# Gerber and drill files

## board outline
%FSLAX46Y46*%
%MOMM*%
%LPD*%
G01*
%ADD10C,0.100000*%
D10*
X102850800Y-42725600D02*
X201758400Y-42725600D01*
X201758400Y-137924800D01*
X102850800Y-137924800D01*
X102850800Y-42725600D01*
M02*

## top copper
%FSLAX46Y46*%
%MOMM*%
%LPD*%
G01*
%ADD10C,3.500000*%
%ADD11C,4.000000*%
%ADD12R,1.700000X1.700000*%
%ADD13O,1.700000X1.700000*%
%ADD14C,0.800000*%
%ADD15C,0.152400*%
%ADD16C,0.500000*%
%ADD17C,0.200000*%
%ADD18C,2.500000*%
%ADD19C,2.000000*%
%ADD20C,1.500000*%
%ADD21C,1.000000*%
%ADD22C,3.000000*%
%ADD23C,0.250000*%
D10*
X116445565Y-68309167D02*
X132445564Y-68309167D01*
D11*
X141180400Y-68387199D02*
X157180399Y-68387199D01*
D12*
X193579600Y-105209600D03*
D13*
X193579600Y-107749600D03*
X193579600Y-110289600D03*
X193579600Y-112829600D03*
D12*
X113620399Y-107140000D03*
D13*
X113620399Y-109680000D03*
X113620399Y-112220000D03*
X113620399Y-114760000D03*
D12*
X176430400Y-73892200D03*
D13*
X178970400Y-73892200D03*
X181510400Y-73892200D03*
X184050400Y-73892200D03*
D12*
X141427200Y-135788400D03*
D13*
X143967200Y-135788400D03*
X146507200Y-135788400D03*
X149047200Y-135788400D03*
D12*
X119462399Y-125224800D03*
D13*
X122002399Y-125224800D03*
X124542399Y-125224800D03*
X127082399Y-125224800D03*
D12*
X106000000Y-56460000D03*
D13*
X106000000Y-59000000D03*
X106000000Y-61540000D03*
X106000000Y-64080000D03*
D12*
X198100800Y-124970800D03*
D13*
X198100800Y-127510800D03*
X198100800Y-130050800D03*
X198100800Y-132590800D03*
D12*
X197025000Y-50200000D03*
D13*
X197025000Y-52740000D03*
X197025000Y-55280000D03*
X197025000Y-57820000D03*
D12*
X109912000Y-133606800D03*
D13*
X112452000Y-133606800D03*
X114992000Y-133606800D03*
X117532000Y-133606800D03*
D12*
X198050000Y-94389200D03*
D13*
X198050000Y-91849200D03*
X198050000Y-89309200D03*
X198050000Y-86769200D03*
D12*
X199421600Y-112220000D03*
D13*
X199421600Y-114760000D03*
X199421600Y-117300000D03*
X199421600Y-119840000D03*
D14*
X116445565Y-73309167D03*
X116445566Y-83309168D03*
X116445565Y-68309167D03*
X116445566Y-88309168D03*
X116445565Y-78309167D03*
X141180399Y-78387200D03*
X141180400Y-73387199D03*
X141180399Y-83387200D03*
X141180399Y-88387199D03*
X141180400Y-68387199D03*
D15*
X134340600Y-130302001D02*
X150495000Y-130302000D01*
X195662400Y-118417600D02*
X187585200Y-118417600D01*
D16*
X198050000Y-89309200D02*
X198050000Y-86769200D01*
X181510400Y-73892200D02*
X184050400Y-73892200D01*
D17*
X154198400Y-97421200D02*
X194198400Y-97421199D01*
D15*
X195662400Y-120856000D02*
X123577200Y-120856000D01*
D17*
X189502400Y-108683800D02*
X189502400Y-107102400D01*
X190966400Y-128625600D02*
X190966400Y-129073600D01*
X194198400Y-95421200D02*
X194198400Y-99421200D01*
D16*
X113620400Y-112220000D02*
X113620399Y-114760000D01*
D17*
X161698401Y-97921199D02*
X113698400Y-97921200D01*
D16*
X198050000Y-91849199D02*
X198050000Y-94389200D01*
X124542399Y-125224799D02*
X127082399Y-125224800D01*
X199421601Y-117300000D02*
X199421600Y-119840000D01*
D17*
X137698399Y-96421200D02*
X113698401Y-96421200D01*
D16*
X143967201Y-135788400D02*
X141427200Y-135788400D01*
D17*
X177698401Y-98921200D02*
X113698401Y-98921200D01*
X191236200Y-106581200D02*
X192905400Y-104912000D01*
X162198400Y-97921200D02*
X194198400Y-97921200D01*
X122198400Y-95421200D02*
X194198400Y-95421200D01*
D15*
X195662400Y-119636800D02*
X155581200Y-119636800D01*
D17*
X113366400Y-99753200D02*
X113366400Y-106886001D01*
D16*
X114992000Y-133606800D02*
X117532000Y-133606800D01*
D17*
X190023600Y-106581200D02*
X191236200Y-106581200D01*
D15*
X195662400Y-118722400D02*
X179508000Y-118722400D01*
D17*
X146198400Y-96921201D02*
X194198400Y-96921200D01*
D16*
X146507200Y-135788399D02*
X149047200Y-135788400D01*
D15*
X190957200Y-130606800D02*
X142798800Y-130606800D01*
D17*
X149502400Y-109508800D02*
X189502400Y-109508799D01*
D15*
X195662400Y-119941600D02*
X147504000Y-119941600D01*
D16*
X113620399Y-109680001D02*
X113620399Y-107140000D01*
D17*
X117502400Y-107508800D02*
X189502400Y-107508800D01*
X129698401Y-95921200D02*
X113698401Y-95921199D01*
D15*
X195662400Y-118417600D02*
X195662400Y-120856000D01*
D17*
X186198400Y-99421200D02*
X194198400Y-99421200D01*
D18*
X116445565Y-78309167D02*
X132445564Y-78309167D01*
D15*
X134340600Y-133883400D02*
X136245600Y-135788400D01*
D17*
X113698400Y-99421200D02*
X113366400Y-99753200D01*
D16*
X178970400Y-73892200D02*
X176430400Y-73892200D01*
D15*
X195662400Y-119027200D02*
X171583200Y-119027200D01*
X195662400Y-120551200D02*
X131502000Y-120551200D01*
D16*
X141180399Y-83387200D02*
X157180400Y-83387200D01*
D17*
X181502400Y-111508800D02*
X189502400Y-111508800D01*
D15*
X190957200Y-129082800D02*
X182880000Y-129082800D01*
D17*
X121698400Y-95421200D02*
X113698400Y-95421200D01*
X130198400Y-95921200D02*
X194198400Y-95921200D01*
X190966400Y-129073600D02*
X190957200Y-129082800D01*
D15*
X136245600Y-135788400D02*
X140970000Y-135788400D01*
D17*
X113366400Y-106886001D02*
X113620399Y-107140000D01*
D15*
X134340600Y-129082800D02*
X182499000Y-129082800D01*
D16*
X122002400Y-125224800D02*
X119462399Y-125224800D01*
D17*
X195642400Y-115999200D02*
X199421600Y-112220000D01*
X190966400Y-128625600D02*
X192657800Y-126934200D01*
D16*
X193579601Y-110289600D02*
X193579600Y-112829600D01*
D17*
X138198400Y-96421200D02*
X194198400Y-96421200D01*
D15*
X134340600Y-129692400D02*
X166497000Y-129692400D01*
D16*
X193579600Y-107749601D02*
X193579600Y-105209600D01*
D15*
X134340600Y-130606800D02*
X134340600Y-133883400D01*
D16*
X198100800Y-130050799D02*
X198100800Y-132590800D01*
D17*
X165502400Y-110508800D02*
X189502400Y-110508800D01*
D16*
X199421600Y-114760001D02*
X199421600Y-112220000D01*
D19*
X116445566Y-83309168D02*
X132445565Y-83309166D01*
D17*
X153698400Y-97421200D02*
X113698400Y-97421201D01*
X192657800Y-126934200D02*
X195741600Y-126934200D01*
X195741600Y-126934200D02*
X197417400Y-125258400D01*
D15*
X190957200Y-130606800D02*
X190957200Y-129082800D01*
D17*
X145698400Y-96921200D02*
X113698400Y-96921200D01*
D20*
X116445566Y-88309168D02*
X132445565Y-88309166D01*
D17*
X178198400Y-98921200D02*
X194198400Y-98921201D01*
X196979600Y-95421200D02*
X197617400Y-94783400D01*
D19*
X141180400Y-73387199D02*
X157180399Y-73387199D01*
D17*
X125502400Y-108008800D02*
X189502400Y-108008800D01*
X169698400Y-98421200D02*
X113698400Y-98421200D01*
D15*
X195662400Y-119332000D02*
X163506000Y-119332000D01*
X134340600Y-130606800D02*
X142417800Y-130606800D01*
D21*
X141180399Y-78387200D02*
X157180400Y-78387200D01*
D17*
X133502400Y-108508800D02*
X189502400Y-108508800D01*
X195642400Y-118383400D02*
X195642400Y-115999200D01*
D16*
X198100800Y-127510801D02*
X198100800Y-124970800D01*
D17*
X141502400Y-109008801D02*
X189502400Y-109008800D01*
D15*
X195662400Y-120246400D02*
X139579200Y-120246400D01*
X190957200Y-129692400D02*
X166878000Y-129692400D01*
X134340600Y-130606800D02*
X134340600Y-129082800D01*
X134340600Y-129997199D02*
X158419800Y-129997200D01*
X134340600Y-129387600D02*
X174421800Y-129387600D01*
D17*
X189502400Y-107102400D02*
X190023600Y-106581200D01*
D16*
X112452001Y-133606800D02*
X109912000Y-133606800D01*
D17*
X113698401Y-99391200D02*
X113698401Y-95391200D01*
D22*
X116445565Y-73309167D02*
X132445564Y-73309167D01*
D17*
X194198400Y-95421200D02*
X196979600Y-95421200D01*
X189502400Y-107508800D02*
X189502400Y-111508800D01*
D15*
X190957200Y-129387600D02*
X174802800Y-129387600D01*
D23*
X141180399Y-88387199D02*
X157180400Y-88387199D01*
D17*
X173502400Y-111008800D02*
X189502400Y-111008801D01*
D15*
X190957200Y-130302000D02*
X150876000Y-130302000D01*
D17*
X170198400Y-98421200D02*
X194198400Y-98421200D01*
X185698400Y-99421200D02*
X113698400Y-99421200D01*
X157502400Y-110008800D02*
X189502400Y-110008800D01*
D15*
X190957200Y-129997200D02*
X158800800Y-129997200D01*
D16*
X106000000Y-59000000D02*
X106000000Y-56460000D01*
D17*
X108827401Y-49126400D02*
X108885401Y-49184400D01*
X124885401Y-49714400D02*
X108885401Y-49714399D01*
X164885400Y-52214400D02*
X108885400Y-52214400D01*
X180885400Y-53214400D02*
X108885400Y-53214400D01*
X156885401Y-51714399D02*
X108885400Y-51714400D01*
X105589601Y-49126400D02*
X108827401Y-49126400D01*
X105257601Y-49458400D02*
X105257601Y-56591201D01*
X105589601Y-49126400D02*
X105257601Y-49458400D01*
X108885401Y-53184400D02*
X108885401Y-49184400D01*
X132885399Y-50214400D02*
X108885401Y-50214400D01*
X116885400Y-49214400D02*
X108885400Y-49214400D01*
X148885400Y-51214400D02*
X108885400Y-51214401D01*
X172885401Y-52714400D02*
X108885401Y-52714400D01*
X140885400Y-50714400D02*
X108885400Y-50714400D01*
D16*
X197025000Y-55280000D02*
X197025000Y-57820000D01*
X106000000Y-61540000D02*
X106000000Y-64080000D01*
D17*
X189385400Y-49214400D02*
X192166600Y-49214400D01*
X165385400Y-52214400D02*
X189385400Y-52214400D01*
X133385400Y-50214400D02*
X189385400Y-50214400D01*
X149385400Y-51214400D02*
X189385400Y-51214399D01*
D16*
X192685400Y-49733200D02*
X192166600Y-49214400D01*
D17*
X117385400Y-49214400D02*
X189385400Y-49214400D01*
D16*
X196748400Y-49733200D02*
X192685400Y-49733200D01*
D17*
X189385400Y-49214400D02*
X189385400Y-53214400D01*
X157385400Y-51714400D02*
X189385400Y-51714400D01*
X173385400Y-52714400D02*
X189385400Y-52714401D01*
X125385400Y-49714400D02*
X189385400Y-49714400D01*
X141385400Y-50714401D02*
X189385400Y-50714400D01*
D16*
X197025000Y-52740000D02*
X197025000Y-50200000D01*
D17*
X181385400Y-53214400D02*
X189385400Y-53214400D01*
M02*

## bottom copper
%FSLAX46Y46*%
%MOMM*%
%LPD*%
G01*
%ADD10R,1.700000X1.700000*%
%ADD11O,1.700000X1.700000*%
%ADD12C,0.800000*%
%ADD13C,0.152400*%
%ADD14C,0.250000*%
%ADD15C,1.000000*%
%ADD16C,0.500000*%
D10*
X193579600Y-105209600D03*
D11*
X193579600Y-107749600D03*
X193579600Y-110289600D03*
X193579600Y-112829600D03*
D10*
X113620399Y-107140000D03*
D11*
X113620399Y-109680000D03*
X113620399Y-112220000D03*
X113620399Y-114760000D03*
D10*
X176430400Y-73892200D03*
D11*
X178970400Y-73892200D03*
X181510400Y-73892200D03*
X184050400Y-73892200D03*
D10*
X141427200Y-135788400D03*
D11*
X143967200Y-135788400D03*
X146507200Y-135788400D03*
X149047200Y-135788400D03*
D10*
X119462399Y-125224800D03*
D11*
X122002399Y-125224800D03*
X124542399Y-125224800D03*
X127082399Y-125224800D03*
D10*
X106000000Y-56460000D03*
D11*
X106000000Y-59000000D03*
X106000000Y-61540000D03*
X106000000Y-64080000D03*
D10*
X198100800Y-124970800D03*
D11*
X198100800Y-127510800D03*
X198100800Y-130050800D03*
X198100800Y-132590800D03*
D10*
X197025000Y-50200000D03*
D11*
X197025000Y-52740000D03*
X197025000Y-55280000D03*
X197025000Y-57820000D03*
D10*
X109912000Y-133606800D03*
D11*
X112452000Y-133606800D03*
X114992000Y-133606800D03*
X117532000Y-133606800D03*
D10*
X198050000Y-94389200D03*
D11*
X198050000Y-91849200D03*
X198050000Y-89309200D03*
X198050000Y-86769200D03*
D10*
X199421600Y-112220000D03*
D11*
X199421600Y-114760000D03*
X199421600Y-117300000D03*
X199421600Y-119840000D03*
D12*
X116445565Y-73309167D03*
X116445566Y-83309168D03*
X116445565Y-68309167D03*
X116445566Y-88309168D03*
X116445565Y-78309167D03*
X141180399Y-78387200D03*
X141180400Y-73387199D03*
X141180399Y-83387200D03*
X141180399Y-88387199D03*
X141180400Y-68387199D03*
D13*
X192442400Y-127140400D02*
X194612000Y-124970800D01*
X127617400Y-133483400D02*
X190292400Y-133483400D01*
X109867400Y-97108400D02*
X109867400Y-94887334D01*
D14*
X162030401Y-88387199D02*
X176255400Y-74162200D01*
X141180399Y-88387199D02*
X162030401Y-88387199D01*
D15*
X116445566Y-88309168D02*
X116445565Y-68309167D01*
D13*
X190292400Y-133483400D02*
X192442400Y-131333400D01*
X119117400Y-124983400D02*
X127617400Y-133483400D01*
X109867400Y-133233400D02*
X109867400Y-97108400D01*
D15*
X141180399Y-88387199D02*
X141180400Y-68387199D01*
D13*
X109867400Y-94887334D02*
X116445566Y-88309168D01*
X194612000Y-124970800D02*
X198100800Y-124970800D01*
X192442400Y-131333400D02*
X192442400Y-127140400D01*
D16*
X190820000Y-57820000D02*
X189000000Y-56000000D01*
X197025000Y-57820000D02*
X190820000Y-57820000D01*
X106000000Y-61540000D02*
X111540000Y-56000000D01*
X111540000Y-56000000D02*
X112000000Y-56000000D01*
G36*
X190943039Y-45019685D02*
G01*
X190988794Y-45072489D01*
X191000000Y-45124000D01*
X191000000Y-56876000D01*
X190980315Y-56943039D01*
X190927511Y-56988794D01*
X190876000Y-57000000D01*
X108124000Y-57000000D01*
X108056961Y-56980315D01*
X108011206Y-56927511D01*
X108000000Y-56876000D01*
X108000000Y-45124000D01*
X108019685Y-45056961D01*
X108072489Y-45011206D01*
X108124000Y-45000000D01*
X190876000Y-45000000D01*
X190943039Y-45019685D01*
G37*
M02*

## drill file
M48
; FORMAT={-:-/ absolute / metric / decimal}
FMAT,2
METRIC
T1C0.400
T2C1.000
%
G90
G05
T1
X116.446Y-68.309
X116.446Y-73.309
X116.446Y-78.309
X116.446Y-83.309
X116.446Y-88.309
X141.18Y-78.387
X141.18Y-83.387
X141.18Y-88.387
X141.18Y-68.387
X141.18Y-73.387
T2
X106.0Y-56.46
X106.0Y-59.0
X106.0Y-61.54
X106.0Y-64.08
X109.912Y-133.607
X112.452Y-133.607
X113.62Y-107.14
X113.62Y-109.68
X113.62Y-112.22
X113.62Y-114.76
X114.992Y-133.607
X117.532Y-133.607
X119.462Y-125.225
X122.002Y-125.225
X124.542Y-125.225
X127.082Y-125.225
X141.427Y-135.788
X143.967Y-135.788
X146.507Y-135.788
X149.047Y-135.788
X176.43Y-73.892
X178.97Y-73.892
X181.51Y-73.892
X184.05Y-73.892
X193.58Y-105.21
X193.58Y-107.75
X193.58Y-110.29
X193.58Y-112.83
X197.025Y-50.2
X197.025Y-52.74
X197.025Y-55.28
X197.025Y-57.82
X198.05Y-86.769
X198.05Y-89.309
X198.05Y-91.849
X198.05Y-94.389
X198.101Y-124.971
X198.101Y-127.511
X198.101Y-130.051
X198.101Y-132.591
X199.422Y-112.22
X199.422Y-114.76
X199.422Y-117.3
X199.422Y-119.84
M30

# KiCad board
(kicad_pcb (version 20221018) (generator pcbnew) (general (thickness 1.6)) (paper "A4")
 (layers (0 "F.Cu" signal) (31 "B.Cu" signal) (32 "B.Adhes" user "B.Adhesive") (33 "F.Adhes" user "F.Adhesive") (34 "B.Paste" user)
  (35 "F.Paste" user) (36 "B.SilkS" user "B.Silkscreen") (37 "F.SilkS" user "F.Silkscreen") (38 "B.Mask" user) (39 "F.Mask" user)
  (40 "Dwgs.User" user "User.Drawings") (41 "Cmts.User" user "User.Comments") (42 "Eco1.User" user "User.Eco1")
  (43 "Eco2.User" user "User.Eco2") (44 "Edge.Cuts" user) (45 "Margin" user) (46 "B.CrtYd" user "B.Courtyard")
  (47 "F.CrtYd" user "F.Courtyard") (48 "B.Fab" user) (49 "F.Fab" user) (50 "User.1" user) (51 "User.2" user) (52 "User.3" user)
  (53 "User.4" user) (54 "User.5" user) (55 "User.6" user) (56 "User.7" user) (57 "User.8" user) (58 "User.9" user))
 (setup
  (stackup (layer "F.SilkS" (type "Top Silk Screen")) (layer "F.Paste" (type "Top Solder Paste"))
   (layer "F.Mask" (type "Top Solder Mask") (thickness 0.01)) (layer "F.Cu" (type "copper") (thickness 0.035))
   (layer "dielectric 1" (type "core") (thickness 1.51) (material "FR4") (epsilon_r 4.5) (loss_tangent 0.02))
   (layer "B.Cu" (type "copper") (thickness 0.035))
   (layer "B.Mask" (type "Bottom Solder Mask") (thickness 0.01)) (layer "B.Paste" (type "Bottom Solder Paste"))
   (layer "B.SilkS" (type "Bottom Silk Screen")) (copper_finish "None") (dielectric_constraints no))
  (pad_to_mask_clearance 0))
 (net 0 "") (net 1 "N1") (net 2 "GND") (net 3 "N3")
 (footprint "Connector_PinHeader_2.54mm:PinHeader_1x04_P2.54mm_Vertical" (layer "F.Cu") (at 193.5796 105.2096)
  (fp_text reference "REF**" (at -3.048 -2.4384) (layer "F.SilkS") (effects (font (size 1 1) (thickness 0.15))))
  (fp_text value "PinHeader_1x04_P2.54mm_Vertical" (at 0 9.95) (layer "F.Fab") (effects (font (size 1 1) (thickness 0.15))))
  (pad "1" thru_hole rect (at 0 0) (size 1.7 1.7) (drill 1) (layers "*.Cu" "*.Mask"))
  (pad "2" thru_hole oval (at 0 2.54) (size 1.7 1.7) (drill 1) (layers "*.Cu" "*.Mask"))
  (pad "3" thru_hole oval (at 0 5.08) (size 1.7 1.7) (drill 1) (layers "*.Cu" "*.Mask"))
  (pad "4" thru_hole oval (at 0 7.62) (size 1.7 1.7) (drill 1) (layers "*.Cu" "*.Mask")))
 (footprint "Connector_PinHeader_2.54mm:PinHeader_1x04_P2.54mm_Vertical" (layer "F.Cu") (at 113.620399 107.14)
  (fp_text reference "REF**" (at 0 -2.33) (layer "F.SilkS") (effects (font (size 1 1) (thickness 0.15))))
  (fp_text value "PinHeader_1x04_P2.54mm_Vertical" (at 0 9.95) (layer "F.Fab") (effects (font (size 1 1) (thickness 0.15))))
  (pad "1" thru_hole rect (at 0 0) (size 1.7 1.7) (drill 1) (layers "*.Cu" "*.Mask"))
  (pad "2" thru_hole oval (at 0 2.54) (size 1.7 1.7) (drill 1) (layers "*.Cu" "*.Mask"))
  (pad "3" thru_hole oval (at 0 5.08) (size 1.7 1.7) (drill 1) (layers "*.Cu" "*.Mask"))
  (pad "4" thru_hole oval (at 0 7.62) (size 1.7 1.7) (drill 1) (layers "*.Cu" "*.Mask")))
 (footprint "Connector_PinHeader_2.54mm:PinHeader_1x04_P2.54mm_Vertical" (layer "F.Cu") (at 176.4304 73.8922 90)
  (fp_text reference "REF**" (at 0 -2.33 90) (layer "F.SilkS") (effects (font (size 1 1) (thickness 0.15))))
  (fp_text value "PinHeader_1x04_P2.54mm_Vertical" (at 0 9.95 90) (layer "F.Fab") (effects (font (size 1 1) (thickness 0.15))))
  (pad "1" thru_hole rect (at 0 0 90) (size 1.7 1.7) (drill 1) (layers "*.Cu" "*.Mask"))
  (pad "2" thru_hole oval (at 0 2.54 90) (size 1.7 1.7) (drill 1) (layers "*.Cu" "*.Mask"))
  (pad "3" thru_hole oval (at 0 5.08 90) (size 1.7 1.7) (drill 1) (layers "*.Cu" "*.Mask"))
  (pad "4" thru_hole oval (at 0 7.62 90) (size 1.7 1.7) (drill 1) (layers "*.Cu" "*.Mask")))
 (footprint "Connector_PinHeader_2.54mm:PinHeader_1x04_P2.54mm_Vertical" (layer "F.Cu") (at 141.4272 135.7884 90)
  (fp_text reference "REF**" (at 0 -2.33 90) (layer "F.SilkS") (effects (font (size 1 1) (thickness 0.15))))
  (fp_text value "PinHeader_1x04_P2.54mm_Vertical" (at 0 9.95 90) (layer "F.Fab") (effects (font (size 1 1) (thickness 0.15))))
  (pad "1" thru_hole rect (at 0 0 90) (size 1.7 1.7) (drill 1) (layers "*.Cu" "*.Mask"))
  (pad "2" thru_hole oval (at 0 2.54 90) (size 1.7 1.7) (drill 1) (layers "*.Cu" "*.Mask"))
  (pad "3" thru_hole oval (at 0 5.08 90) (size 1.7 1.7) (drill 1) (layers "*.Cu" "*.Mask"))
  (pad "4" thru_hole oval (at 0 7.62 90) (size 1.7 1.7) (drill 1) (layers "*.Cu" "*.Mask")))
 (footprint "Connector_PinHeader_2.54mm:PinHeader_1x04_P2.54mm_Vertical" (layer "F.Cu") (at 119.462399 125.2248 90)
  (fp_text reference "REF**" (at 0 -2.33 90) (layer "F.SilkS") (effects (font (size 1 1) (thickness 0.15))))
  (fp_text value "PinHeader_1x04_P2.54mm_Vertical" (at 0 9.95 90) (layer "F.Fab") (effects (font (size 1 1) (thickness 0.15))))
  (pad "1" thru_hole rect (at 0 0 90) (size 1.7 1.7) (drill 1) (layers "*.Cu" "*.Mask"))
  (pad "2" thru_hole oval (at 0 2.54 90) (size 1.7 1.7) (drill 1) (layers "*.Cu" "*.Mask"))
  (pad "3" thru_hole oval (at 0 5.08 90) (size 1.7 1.7) (drill 1) (layers "*.Cu" "*.Mask"))
  (pad "4" thru_hole oval (at 0 7.62 90) (size 1.7 1.7) (drill 1) (layers "*.Cu" "*.Mask")))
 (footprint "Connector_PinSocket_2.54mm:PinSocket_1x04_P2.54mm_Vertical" (layer "F.Cu") (at 106 56.46)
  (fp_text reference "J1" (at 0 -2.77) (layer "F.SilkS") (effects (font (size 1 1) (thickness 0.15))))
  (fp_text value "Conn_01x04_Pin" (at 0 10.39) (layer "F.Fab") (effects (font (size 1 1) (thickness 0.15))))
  (pad "1" thru_hole rect (at 0 0) (size 1.7 1.7) (drill 1) (layers "*.Cu" "*.Mask") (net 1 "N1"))
  (pad "2" thru_hole oval (at 0 2.54) (size 1.7 1.7) (drill 1) (layers "*.Cu" "*.Mask") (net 1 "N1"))
  (pad "3" thru_hole oval (at 0 5.08) (size 1.7 1.7) (drill 1) (layers "*.Cu" "*.Mask") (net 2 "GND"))
  (pad "4" thru_hole oval (at 0 7.62) (size 1.7 1.7) (drill 1) (layers "*.Cu" "*.Mask") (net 2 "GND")))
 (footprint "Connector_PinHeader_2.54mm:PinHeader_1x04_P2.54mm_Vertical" (layer "F.Cu") (at 198.1008 124.9708)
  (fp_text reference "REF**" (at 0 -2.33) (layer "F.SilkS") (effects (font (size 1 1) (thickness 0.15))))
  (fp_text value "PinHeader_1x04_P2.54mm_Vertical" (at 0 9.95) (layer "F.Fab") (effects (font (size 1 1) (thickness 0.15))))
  (pad "1" thru_hole rect (at 0 0) (size 1.7 1.7) (drill 1) (layers "*.Cu" "*.Mask"))
  (pad "2" thru_hole oval (at 0 2.54) (size 1.7 1.7) (drill 1) (layers "*.Cu" "*.Mask"))
  (pad "3" thru_hole oval (at 0 5.08) (size 1.7 1.7) (drill 1) (layers "*.Cu" "*.Mask"))
  (pad "4" thru_hole oval (at 0 7.62) (size 1.7 1.7) (drill 1) (layers "*.Cu" "*.Mask")))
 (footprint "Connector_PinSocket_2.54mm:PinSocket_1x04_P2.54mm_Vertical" (layer "F.Cu") (at 197.025 50.2)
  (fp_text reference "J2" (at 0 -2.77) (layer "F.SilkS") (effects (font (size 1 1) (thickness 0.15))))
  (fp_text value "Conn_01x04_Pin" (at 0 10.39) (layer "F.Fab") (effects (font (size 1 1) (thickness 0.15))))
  (pad "1" thru_hole rect (at 0 0) (size 1.7 1.7) (drill 1) (layers "*.Cu" "*.Mask") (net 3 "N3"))
  (pad "2" thru_hole oval (at 0 2.54) (size 1.7 1.7) (drill 1) (layers "*.Cu" "*.Mask") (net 3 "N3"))
  (pad "3" thru_hole oval (at 0 5.08) (size 1.7 1.7) (drill 1) (layers "*.Cu" "*.Mask") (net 2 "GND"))
  (pad "4" thru_hole oval (at 0 7.62) (size 1.7 1.7) (drill 1) (layers "*.Cu" "*.Mask") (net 2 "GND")))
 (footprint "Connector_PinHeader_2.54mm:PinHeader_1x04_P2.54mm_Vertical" (layer "F.Cu") (at 109.912 133.6068 90)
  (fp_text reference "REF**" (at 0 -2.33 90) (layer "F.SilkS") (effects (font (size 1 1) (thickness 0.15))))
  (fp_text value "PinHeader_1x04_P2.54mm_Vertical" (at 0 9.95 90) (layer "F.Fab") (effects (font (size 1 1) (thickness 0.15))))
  (pad "1" thru_hole rect (at 0 0 90) (size 1.7 1.7) (drill 1) (layers "*.Cu" "*.Mask"))
  (pad "2" thru_hole oval (at 0 2.54 90) (size 1.7 1.7) (drill 1) (layers "*.Cu" "*.Mask"))
  (pad "3" thru_hole oval (at 0 5.08 90) (size 1.7 1.7) (drill 1) (layers "*.Cu" "*.Mask"))
  (pad "4" thru_hole oval (at 0 7.62 90) (size 1.7 1.7) (drill 1) (layers "*.Cu" "*.Mask")))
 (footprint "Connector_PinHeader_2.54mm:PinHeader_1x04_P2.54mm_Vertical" (layer "F.Cu") (at 198.05 94.3892 180)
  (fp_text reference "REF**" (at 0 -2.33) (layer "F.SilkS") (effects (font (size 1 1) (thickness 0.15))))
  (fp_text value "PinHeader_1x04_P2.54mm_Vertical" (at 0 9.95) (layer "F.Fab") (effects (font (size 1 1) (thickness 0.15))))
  (pad "1" thru_hole rect (at 0 0 180) (size 1.7 1.7) (drill 1) (layers "*.Cu" "*.Mask"))
  (pad "2" thru_hole oval (at 0 2.54 180) (size 1.7 1.7) (drill 1) (layers "*.Cu" "*.Mask"))
  (pad "3" thru_hole oval (at 0 5.08 180) (size 1.7 1.7) (drill 1) (layers "*.Cu" "*.Mask"))
  (pad "4" thru_hole oval (at 0 7.62 180) (size 1.7 1.7) (drill 1) (layers "*.Cu" "*.Mask")))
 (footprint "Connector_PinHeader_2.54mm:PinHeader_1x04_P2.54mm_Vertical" (layer "F.Cu") (at 199.4216 112.22)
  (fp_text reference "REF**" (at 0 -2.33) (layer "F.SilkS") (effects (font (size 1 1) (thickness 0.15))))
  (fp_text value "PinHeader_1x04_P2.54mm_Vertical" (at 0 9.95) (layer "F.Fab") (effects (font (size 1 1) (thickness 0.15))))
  (pad "1" thru_hole rect (at 0 0) (size 1.7 1.7) (drill 1) (layers "*.Cu" "*.Mask"))
  (pad "2" thru_hole oval (at 0 2.54) (size 1.7 1.7) (drill 1) (layers "*.Cu" "*.Mask"))
  (pad "3" thru_hole oval (at 0 5.08) (size 1.7 1.7) (drill 1) (layers "*.Cu" "*.Mask"))
  (pad "4" thru_hole oval (at 0 7.62) (size 1.7 1.7) (drill 1) (layers "*.Cu" "*.Mask")))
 (gr_line (start 116.445565 68.309167) (end 132.445564 68.309167) (stroke (width 3.5) (type default)) (layer "F.Cu"))
 (gr_line (start 141.1804 68.387199) (end 157.180399 68.387199) (stroke (width 4) (type default)) (layer "F.Cu"))
 (gr_rect (start 102.8508 42.7256) (end 201.7584 137.9248) (stroke (width 0.1) (type default)) (fill none) (layer "Edge.Cuts"))
 (segment (start 134.3406 130.302001) (end 150.495 130.302) (width 0.1524) (layer "F.Cu") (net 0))
 (segment (start 195.6624 118.4176) (end 187.5852 118.4176) (width 0.1524) (layer "F.Cu") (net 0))
 (segment (start 198.05 89.3092) (end 198.05 86.7692) (width 0.5) (layer "F.Cu") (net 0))
 (segment (start 181.5104 73.8922) (end 184.0504 73.8922) (width 0.5) (layer "F.Cu") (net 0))
 (segment (start 154.1984 97.4212) (end 194.1984 97.421199) (width 0.2) (layer "F.Cu") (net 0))
 (segment (start 195.6624 120.856) (end 123.5772 120.856) (width 0.1524) (layer "F.Cu") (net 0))
 (segment (start 189.5024 108.6838) (end 189.5024 107.1024) (width 0.2) (layer "F.Cu") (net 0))
 (segment (start 190.9664 128.6256) (end 190.9664 129.0736) (width 0.2) (layer "F.Cu") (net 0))
 (segment (start 194.1984 95.4212) (end 194.1984 99.4212) (width 0.2) (layer "F.Cu") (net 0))
 (segment (start 113.6204 112.22) (end 113.620399 114.76) (width 0.5) (layer "F.Cu") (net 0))
 (segment (start 161.698401 97.921199) (end 113.6984 97.9212) (width 0.2) (layer "F.Cu") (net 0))
 (segment (start 198.05 91.849199) (end 198.05 94.3892) (width 0.5) (layer "F.Cu") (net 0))
 (segment (start 124.542399 125.224799) (end 127.082399 125.2248) (width 0.5) (layer "F.Cu") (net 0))
 (segment (start 199.421601 117.3) (end 199.4216 119.84) (width 0.5) (layer "F.Cu") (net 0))
 (segment (start 137.698399 96.4212) (end 113.698401 96.4212) (width 0.2) (layer "F.Cu") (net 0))
 (segment (start 143.967201 135.7884) (end 141.4272 135.7884) (width 0.5) (layer "F.Cu") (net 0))
 (segment (start 177.698401 98.9212) (end 113.698401 98.9212) (width 0.2) (layer "F.Cu") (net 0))
 (segment (start 191.2362 106.5812) (end 192.9054 104.912) (width 0.2) (layer "F.Cu") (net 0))
 (segment (start 162.1984 97.9212) (end 194.1984 97.9212) (width 0.2) (layer "F.Cu") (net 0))
 (segment (start 122.1984 95.4212) (end 194.1984 95.4212) (width 0.2) (layer "F.Cu") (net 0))
 (segment (start 195.6624 119.6368) (end 155.5812 119.6368) (width 0.1524) (layer "F.Cu") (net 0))
 (segment (start 113.3664 99.7532) (end 113.3664 106.886001) (width 0.2) (layer "F.Cu") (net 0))
 (segment (start 114.992 133.6068) (end 117.532 133.6068) (width 0.5) (layer "F.Cu") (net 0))
 (segment (start 190.0236 106.5812) (end 191.2362 106.5812) (width 0.2) (layer "F.Cu") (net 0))
 (segment (start 195.6624 118.7224) (end 179.508 118.7224) (width 0.1524) (layer "F.Cu") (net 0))
 (segment (start 146.1984 96.921201) (end 194.1984 96.9212) (width 0.2) (layer "F.Cu") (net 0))
 (segment (start 146.5072 135.788399) (end 149.0472 135.7884) (width 0.5) (layer "F.Cu") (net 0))
 (segment (start 190.9572 130.6068) (end 142.7988 130.6068) (width 0.1524) (layer "F.Cu") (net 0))
 (segment (start 149.5024 109.5088) (end 189.5024 109.508799) (width 0.2) (layer "F.Cu") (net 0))
 (segment (start 195.6624 119.9416) (end 147.504 119.9416) (width 0.1524) (layer "F.Cu") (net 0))
 (segment (start 113.620399 109.680001) (end 113.620399 107.14) (width 0.5) (layer "F.Cu") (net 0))
 (segment (start 117.5024 107.5088) (end 189.5024 107.5088) (width 0.2) (layer "F.Cu") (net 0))
 (segment (start 129.698401 95.9212) (end 113.698401 95.921199) (width 0.2) (layer "F.Cu") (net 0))
 (segment (start 195.6624 118.4176) (end 195.6624 120.856) (width 0.1524) (layer "F.Cu") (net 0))
 (segment (start 186.1984 99.4212) (end 194.1984 99.4212) (width 0.2) (layer "F.Cu") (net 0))
 (segment (start 116.445565 78.309167) (end 132.445564 78.309167) (width 2.5) (layer "F.Cu") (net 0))
 (segment (start 134.3406 133.8834) (end 136.2456 135.7884) (width 0.1524) (layer "F.Cu") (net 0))
 (segment (start 113.6984 99.4212) (end 113.3664 99.7532) (width 0.2) (layer "F.Cu") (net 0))
 (segment (start 178.9704 73.8922) (end 176.4304 73.8922) (width 0.5) (layer "F.Cu") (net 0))
 (segment (start 195.6624 119.0272) (end 171.5832 119.0272) (width 0.1524) (layer "F.Cu") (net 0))
 (segment (start 195.6624 120.5512) (end 131.502 120.5512) (width 0.1524) (layer "F.Cu") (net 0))
 (segment (start 141.180399 83.3872) (end 157.1804 83.3872) (width 0.5) (layer "F.Cu") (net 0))
 (segment (start 181.5024 111.5088) (end 189.5024 111.5088) (width 0.2) (layer "F.Cu") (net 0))
 (segment (start 190.9572 129.0828) (end 182.88 129.0828) (width 0.1524) (layer "F.Cu") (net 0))
 (segment (start 121.6984 95.4212) (end 113.6984 95.4212) (width 0.2) (layer "F.Cu") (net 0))
 (segment (start 130.1984 95.9212) (end 194.1984 95.9212) (width 0.2) (layer "F.Cu") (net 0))
 (segment (start 190.9664 129.0736) (end 190.9572 129.0828) (width 0.2) (layer "F.Cu") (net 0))
 (segment (start 136.2456 135.7884) (end 140.97 135.7884) (width 0.1524) (layer "F.Cu") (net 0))
 (segment (start 113.3664 106.886001) (end 113.620399 107.14) (width 0.2) (layer "F.Cu") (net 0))
 (segment (start 134.3406 129.0828) (end 182.499 129.0828) (width 0.1524) (layer "F.Cu") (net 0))
 (segment (start 122.0024 125.2248) (end 119.462399 125.2248) (width 0.5) (layer "F.Cu") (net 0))
 (segment (start 195.6424 115.9992) (end 199.4216 112.22) (width 0.2) (layer "F.Cu") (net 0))
 (segment (start 190.9664 128.6256) (end 192.6578 126.9342) (width 0.2) (layer "F.Cu") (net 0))
 (segment (start 193.579601 110.2896) (end 193.5796 112.8296) (width 0.5) (layer "F.Cu") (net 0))
 (segment (start 138.1984 96.4212) (end 194.1984 96.4212) (width 0.2) (layer "F.Cu") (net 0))
 (segment (start 134.3406 129.6924) (end 166.497 129.6924) (width 0.1524) (layer "F.Cu") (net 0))
 (segment (start 193.5796 107.749601) (end 193.5796 105.2096) (width 0.5) (layer "F.Cu") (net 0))
 (segment (start 134.3406 130.6068) (end 134.3406 133.8834) (width 0.1524) (layer "F.Cu") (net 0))
 (segment (start 198.1008 130.050799) (end 198.1008 132.5908) (width 0.5) (layer "F.Cu") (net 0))
 (segment (start 165.5024 110.5088) (end 189.5024 110.5088) (width 0.2) (layer "F.Cu") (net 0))
 (segment (start 199.4216 114.760001) (end 199.4216 112.22) (width 0.5) (layer "F.Cu") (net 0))
 (segment (start 116.445566 83.309168) (end 132.445565 83.309166) (width 2) (layer "F.Cu") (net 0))
 (segment (start 153.6984 97.4212) (end 113.6984 97.421201) (width 0.2) (layer "F.Cu") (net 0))
 (segment (start 192.6578 126.9342) (end 195.7416 126.9342) (width 0.2) (layer "F.Cu") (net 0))
 (segment (start 195.7416 126.9342) (end 197.4174 125.2584) (width 0.2) (layer "F.Cu") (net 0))
 (segment (start 190.9572 130.6068) (end 190.9572 129.0828) (width 0.1524) (layer "F.Cu") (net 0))
 (segment (start 145.6984 96.9212) (end 113.6984 96.9212) (width 0.2) (layer "F.Cu") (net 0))
 (segment (start 116.445566 88.309168) (end 132.445565 88.309166) (width 1.5) (layer "F.Cu") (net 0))
 (segment (start 178.1984 98.9212) (end 194.1984 98.921201) (width 0.2) (layer "F.Cu") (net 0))
 (segment (start 196.9796 95.4212) (end 197.6174 94.7834) (width 0.2) (layer "F.Cu") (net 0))
 (segment (start 141.1804 73.387199) (end 157.180399 73.387199) (width 2) (layer "F.Cu") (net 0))
 (segment (start 125.5024 108.0088) (end 189.5024 108.0088) (width 0.2) (layer "F.Cu") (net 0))
 (segment (start 169.6984 98.4212) (end 113.6984 98.4212) (width 0.2) (layer "F.Cu") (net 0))
 (segment (start 195.6624 119.332) (end 163.506 119.332) (width 0.1524) (layer "F.Cu") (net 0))
 (segment (start 134.3406 130.6068) (end 142.4178 130.6068) (width 0.1524) (layer "F.Cu") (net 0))
 (segment (start 141.180399 78.3872) (end 157.1804 78.3872) (width 1) (layer "F.Cu") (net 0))
 (segment (start 133.5024 108.5088) (end 189.5024 108.5088) (width 0.2) (layer "F.Cu") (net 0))
 (segment (start 195.6424 118.3834) (end 195.6424 115.9992) (width 0.2) (layer "F.Cu") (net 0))
 (segment (start 198.1008 127.510801) (end 198.1008 124.9708) (width 0.5) (layer "F.Cu") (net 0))
 (segment (start 141.5024 109.008801) (end 189.5024 109.0088) (width 0.2) (layer "F.Cu") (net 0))
 (segment (start 195.6624 120.2464) (end 139.5792 120.2464) (width 0.1524) (layer "F.Cu") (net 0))
 (segment (start 190.9572 129.6924) (end 166.878 129.6924) (width 0.1524) (layer "F.Cu") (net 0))
 (segment (start 134.3406 130.6068) (end 134.3406 129.0828) (width 0.1524) (layer "F.Cu") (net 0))
 (segment (start 134.3406 129.997199) (end 158.4198 129.9972) (width 0.1524) (layer "F.Cu") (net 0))
 (segment (start 134.3406 129.3876) (end 174.4218 129.3876) (width 0.1524) (layer "F.Cu") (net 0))
 (segment (start 189.5024 107.1024) (end 190.0236 106.5812) (width 0.2) (layer "F.Cu") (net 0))
 (segment (start 112.452001 133.6068) (end 109.912 133.6068) (width 0.5) (layer "F.Cu") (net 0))
 (segment (start 113.698401 99.3912) (end 113.698401 95.3912) (width 0.2) (layer "F.Cu") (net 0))
 (segment (start 116.445565 73.309167) (end 132.445564 73.309167) (width 3) (layer "F.Cu") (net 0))
 (segment (start 194.1984 95.4212) (end 196.9796 95.4212) (width 0.2) (layer "F.Cu") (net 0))
 (segment (start 189.5024 107.5088) (end 189.5024 111.5088) (width 0.2) (layer "F.Cu") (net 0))
 (segment (start 190.9572 129.3876) (end 174.8028 129.3876) (width 0.1524) (layer "F.Cu") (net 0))
 (segment (start 141.180399 88.387199) (end 157.1804 88.387199) (width 0.25) (layer "F.Cu") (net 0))
 (segment (start 173.5024 111.0088) (end 189.5024 111.008801) (width 0.2) (layer "F.Cu") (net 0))
 (segment (start 190.9572 130.302) (end 150.876 130.302) (width 0.1524) (layer "F.Cu") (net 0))
 (segment (start 170.1984 98.4212) (end 194.1984 98.4212) (width 0.2) (layer "F.Cu") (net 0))
 (segment (start 185.6984 99.4212) (end 113.6984 99.4212) (width 0.2) (layer "F.Cu") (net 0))
 (segment (start 157.5024 110.0088) (end 189.5024 110.0088) (width 0.2) (layer "F.Cu") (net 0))
 (segment (start 190.9572 129.9972) (end 158.8008 129.9972) (width 0.1524) (layer "F.Cu") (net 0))
 (via (at 116.445565 73.309167) (size 0.8) (drill 0.4) (layers "F.Cu" "B.Cu") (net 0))
 (via (at 116.445566 83.309168) (size 0.8) (drill 0.4) (layers "F.Cu" "B.Cu") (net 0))
 (via (at 116.445565 68.309167) (size 0.8) (drill 0.4) (layers "F.Cu" "B.Cu") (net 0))
 (via (at 116.445566 88.309168) (size 0.8) (drill 0.4) (layers "F.Cu" "B.Cu") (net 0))
 (via (at 116.445565 78.309167) (size 0.8) (drill 0.4) (layers "F.Cu" "B.Cu") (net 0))
 (via (at 141.180399 78.3872) (size 0.8) (drill 0.4) (layers "F.Cu" "B.Cu") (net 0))
 (via (at 141.1804 73.387199) (size 0.8) (drill 0.4) (layers "F.Cu" "B.Cu") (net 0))
 (via (at 141.180399 83.3872) (size 0.8) (drill 0.4) (layers "F.Cu" "B.Cu") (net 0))
 (via (at 141.180399 88.387199) (size 0.8) (drill 0.4) (layers "F.Cu" "B.Cu") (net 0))
 (via (at 141.1804 68.387199) (size 0.8) (drill 0.4) (layers "F.Cu" "B.Cu") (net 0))
 (segment (start 192.4424 127.1404) (end 194.612 124.9708) (width 0.1524) (layer "B.Cu") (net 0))
 (segment (start 127.6174 133.4834) (end 190.2924 133.4834) (width 0.1524) (layer "B.Cu") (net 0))
 (segment (start 109.8674 97.1084) (end 109.8674 94.887334) (width 0.1524) (layer "B.Cu") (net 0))
 (segment (start 162.030401 88.387199) (end 176.2554 74.1622) (width 0.25) (layer "B.Cu") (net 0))
 (segment (start 141.180399 88.387199) (end 162.030401 88.387199) (width 0.25) (layer "B.Cu") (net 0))
 (segment (start 116.445566 88.309168) (end 116.445565 68.309167) (width 1) (layer "B.Cu") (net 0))
 (segment (start 190.2924 133.4834) (end 192.4424 131.3334) (width 0.1524) (layer "B.Cu") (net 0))
 (segment (start 119.1174 124.9834) (end 127.6174 133.4834) (width 0.1524) (layer "B.Cu") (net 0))
 (segment (start 109.8674 133.2334) (end 109.8674 97.1084) (width 0.1524) (layer "B.Cu") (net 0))
 (segment (start 141.180399 88.387199) (end 141.1804 68.387199) (width 1) (layer "B.Cu") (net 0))
 (segment (start 109.8674 94.887334) (end 116.445566 88.309168) (width 0.1524) (layer "B.Cu") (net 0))
 (segment (start 194.612 124.9708) (end 198.1008 124.9708) (width 0.1524) (layer "B.Cu") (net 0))
 (segment (start 192.4424 131.3334) (end 192.4424 127.1404) (width 0.1524) (layer "B.Cu") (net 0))
 (segment (start 106 59) (end 106 56.46) (width 0.5) (layer "F.Cu") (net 1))
 (segment (start 108.827401 49.1264) (end 108.885401 49.1844) (width 0.2) (layer "F.Cu") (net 1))
 (segment (start 124.885401 49.7144) (end 108.885401 49.714399) (width 0.2) (layer "F.Cu") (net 1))
 (segment (start 164.8854 52.2144) (end 108.8854 52.2144) (width 0.2) (layer "F.Cu") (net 1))
 (segment (start 180.8854 53.2144) (end 108.8854 53.2144) (width 0.2) (layer "F.Cu") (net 1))
 (segment (start 156.885401 51.714399) (end 108.8854 51.7144) (width 0.2) (layer "F.Cu") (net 1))
 (segment (start 105.589601 49.1264) (end 108.827401 49.1264) (width 0.2) (layer "F.Cu") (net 1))
 (segment (start 105.257601 49.4584) (end 105.257601 56.591201) (width 0.2) (layer "F.Cu") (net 1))
 (segment (start 105.589601 49.1264) (end 105.257601 49.4584) (width 0.2) (layer "F.Cu") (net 1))
 (segment (start 108.885401 53.1844) (end 108.885401 49.1844) (width 0.2) (layer "F.Cu") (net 1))
 (segment (start 132.885399 50.2144) (end 108.885401 50.2144) (width 0.2) (layer "F.Cu") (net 1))
 (segment (start 116.8854 49.2144) (end 108.8854 49.2144) (width 0.2) (layer "F.Cu") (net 1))
 (segment (start 148.8854 51.2144) (end 108.8854 51.214401) (width 0.2) (layer "F.Cu") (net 1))
 (segment (start 172.885401 52.7144) (end 108.885401 52.7144) (width 0.2) (layer "F.Cu") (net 1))
 (segment (start 140.8854 50.7144) (end 108.8854 50.7144) (width 0.2) (layer "F.Cu") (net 1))
 (segment (start 197.025 55.28) (end 197.025 57.82) (width 0.5) (layer "F.Cu") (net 2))
 (segment (start 106 61.54) (end 106 64.08) (width 0.5) (layer "F.Cu") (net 2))
 (segment (start 190.82 57.82) (end 189 56) (width 0.5) (layer "B.Cu") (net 2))
 (segment (start 197.025 57.82) (end 190.82 57.82) (width 0.5) (layer "B.Cu") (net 2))
 (segment (start 106 61.54) (end 111.54 56) (width 0.5) (layer "B.Cu") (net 2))
 (segment (start 111.54 56) (end 112 56) (width 0.5) (layer "B.Cu") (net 2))
 (segment (start 189.3854 49.2144) (end 192.1666 49.2144) (width 0.2) (layer "F.Cu") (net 3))
 (segment (start 165.3854 52.2144) (end 189.3854 52.2144) (width 0.2) (layer "F.Cu") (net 3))
 (segment (start 133.3854 50.2144) (end 189.3854 50.2144) (width 0.2) (layer "F.Cu") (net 3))
 (segment (start 149.3854 51.2144) (end 189.3854 51.214399) (width 0.2) (layer "F.Cu") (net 3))
 (segment (start 192.6854 49.7332) (end 192.1666 49.2144) (width 0.5) (layer "F.Cu") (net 3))
 (segment (start 117.3854 49.2144) (end 189.3854 49.2144) (width 0.2) (layer "F.Cu") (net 3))
 (segment (start 196.7484 49.7332) (end 192.6854 49.7332) (width 0.5) (layer "F.Cu") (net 3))
 (segment (start 189.3854 49.2144) (end 189.3854 53.2144) (width 0.2) (layer "F.Cu") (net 3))
 (segment (start 157.3854 51.7144) (end 189.3854 51.7144) (width 0.2) (layer "F.Cu") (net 3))
 (segment (start 173.3854 52.7144) (end 189.3854 52.714401) (width 0.2) (layer "F.Cu") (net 3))
 (segment (start 125.3854 49.7144) (end 189.3854 49.7144) (width 0.2) (layer "F.Cu") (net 3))
 (segment (start 141.3854 50.714401) (end 189.3854 50.7144) (width 0.2) (layer "F.Cu") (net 3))
 (segment (start 197.025 52.74) (end 197.025 50.2) (width 0.5) (layer "F.Cu") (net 3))
 (segment (start 181.3854 53.2144) (end 189.3854 53.2144) (width 0.2) (layer "F.Cu") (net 3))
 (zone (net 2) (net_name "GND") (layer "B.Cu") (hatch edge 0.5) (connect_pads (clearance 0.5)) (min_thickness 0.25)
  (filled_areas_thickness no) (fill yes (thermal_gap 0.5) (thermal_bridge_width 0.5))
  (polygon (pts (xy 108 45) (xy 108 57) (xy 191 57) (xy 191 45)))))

